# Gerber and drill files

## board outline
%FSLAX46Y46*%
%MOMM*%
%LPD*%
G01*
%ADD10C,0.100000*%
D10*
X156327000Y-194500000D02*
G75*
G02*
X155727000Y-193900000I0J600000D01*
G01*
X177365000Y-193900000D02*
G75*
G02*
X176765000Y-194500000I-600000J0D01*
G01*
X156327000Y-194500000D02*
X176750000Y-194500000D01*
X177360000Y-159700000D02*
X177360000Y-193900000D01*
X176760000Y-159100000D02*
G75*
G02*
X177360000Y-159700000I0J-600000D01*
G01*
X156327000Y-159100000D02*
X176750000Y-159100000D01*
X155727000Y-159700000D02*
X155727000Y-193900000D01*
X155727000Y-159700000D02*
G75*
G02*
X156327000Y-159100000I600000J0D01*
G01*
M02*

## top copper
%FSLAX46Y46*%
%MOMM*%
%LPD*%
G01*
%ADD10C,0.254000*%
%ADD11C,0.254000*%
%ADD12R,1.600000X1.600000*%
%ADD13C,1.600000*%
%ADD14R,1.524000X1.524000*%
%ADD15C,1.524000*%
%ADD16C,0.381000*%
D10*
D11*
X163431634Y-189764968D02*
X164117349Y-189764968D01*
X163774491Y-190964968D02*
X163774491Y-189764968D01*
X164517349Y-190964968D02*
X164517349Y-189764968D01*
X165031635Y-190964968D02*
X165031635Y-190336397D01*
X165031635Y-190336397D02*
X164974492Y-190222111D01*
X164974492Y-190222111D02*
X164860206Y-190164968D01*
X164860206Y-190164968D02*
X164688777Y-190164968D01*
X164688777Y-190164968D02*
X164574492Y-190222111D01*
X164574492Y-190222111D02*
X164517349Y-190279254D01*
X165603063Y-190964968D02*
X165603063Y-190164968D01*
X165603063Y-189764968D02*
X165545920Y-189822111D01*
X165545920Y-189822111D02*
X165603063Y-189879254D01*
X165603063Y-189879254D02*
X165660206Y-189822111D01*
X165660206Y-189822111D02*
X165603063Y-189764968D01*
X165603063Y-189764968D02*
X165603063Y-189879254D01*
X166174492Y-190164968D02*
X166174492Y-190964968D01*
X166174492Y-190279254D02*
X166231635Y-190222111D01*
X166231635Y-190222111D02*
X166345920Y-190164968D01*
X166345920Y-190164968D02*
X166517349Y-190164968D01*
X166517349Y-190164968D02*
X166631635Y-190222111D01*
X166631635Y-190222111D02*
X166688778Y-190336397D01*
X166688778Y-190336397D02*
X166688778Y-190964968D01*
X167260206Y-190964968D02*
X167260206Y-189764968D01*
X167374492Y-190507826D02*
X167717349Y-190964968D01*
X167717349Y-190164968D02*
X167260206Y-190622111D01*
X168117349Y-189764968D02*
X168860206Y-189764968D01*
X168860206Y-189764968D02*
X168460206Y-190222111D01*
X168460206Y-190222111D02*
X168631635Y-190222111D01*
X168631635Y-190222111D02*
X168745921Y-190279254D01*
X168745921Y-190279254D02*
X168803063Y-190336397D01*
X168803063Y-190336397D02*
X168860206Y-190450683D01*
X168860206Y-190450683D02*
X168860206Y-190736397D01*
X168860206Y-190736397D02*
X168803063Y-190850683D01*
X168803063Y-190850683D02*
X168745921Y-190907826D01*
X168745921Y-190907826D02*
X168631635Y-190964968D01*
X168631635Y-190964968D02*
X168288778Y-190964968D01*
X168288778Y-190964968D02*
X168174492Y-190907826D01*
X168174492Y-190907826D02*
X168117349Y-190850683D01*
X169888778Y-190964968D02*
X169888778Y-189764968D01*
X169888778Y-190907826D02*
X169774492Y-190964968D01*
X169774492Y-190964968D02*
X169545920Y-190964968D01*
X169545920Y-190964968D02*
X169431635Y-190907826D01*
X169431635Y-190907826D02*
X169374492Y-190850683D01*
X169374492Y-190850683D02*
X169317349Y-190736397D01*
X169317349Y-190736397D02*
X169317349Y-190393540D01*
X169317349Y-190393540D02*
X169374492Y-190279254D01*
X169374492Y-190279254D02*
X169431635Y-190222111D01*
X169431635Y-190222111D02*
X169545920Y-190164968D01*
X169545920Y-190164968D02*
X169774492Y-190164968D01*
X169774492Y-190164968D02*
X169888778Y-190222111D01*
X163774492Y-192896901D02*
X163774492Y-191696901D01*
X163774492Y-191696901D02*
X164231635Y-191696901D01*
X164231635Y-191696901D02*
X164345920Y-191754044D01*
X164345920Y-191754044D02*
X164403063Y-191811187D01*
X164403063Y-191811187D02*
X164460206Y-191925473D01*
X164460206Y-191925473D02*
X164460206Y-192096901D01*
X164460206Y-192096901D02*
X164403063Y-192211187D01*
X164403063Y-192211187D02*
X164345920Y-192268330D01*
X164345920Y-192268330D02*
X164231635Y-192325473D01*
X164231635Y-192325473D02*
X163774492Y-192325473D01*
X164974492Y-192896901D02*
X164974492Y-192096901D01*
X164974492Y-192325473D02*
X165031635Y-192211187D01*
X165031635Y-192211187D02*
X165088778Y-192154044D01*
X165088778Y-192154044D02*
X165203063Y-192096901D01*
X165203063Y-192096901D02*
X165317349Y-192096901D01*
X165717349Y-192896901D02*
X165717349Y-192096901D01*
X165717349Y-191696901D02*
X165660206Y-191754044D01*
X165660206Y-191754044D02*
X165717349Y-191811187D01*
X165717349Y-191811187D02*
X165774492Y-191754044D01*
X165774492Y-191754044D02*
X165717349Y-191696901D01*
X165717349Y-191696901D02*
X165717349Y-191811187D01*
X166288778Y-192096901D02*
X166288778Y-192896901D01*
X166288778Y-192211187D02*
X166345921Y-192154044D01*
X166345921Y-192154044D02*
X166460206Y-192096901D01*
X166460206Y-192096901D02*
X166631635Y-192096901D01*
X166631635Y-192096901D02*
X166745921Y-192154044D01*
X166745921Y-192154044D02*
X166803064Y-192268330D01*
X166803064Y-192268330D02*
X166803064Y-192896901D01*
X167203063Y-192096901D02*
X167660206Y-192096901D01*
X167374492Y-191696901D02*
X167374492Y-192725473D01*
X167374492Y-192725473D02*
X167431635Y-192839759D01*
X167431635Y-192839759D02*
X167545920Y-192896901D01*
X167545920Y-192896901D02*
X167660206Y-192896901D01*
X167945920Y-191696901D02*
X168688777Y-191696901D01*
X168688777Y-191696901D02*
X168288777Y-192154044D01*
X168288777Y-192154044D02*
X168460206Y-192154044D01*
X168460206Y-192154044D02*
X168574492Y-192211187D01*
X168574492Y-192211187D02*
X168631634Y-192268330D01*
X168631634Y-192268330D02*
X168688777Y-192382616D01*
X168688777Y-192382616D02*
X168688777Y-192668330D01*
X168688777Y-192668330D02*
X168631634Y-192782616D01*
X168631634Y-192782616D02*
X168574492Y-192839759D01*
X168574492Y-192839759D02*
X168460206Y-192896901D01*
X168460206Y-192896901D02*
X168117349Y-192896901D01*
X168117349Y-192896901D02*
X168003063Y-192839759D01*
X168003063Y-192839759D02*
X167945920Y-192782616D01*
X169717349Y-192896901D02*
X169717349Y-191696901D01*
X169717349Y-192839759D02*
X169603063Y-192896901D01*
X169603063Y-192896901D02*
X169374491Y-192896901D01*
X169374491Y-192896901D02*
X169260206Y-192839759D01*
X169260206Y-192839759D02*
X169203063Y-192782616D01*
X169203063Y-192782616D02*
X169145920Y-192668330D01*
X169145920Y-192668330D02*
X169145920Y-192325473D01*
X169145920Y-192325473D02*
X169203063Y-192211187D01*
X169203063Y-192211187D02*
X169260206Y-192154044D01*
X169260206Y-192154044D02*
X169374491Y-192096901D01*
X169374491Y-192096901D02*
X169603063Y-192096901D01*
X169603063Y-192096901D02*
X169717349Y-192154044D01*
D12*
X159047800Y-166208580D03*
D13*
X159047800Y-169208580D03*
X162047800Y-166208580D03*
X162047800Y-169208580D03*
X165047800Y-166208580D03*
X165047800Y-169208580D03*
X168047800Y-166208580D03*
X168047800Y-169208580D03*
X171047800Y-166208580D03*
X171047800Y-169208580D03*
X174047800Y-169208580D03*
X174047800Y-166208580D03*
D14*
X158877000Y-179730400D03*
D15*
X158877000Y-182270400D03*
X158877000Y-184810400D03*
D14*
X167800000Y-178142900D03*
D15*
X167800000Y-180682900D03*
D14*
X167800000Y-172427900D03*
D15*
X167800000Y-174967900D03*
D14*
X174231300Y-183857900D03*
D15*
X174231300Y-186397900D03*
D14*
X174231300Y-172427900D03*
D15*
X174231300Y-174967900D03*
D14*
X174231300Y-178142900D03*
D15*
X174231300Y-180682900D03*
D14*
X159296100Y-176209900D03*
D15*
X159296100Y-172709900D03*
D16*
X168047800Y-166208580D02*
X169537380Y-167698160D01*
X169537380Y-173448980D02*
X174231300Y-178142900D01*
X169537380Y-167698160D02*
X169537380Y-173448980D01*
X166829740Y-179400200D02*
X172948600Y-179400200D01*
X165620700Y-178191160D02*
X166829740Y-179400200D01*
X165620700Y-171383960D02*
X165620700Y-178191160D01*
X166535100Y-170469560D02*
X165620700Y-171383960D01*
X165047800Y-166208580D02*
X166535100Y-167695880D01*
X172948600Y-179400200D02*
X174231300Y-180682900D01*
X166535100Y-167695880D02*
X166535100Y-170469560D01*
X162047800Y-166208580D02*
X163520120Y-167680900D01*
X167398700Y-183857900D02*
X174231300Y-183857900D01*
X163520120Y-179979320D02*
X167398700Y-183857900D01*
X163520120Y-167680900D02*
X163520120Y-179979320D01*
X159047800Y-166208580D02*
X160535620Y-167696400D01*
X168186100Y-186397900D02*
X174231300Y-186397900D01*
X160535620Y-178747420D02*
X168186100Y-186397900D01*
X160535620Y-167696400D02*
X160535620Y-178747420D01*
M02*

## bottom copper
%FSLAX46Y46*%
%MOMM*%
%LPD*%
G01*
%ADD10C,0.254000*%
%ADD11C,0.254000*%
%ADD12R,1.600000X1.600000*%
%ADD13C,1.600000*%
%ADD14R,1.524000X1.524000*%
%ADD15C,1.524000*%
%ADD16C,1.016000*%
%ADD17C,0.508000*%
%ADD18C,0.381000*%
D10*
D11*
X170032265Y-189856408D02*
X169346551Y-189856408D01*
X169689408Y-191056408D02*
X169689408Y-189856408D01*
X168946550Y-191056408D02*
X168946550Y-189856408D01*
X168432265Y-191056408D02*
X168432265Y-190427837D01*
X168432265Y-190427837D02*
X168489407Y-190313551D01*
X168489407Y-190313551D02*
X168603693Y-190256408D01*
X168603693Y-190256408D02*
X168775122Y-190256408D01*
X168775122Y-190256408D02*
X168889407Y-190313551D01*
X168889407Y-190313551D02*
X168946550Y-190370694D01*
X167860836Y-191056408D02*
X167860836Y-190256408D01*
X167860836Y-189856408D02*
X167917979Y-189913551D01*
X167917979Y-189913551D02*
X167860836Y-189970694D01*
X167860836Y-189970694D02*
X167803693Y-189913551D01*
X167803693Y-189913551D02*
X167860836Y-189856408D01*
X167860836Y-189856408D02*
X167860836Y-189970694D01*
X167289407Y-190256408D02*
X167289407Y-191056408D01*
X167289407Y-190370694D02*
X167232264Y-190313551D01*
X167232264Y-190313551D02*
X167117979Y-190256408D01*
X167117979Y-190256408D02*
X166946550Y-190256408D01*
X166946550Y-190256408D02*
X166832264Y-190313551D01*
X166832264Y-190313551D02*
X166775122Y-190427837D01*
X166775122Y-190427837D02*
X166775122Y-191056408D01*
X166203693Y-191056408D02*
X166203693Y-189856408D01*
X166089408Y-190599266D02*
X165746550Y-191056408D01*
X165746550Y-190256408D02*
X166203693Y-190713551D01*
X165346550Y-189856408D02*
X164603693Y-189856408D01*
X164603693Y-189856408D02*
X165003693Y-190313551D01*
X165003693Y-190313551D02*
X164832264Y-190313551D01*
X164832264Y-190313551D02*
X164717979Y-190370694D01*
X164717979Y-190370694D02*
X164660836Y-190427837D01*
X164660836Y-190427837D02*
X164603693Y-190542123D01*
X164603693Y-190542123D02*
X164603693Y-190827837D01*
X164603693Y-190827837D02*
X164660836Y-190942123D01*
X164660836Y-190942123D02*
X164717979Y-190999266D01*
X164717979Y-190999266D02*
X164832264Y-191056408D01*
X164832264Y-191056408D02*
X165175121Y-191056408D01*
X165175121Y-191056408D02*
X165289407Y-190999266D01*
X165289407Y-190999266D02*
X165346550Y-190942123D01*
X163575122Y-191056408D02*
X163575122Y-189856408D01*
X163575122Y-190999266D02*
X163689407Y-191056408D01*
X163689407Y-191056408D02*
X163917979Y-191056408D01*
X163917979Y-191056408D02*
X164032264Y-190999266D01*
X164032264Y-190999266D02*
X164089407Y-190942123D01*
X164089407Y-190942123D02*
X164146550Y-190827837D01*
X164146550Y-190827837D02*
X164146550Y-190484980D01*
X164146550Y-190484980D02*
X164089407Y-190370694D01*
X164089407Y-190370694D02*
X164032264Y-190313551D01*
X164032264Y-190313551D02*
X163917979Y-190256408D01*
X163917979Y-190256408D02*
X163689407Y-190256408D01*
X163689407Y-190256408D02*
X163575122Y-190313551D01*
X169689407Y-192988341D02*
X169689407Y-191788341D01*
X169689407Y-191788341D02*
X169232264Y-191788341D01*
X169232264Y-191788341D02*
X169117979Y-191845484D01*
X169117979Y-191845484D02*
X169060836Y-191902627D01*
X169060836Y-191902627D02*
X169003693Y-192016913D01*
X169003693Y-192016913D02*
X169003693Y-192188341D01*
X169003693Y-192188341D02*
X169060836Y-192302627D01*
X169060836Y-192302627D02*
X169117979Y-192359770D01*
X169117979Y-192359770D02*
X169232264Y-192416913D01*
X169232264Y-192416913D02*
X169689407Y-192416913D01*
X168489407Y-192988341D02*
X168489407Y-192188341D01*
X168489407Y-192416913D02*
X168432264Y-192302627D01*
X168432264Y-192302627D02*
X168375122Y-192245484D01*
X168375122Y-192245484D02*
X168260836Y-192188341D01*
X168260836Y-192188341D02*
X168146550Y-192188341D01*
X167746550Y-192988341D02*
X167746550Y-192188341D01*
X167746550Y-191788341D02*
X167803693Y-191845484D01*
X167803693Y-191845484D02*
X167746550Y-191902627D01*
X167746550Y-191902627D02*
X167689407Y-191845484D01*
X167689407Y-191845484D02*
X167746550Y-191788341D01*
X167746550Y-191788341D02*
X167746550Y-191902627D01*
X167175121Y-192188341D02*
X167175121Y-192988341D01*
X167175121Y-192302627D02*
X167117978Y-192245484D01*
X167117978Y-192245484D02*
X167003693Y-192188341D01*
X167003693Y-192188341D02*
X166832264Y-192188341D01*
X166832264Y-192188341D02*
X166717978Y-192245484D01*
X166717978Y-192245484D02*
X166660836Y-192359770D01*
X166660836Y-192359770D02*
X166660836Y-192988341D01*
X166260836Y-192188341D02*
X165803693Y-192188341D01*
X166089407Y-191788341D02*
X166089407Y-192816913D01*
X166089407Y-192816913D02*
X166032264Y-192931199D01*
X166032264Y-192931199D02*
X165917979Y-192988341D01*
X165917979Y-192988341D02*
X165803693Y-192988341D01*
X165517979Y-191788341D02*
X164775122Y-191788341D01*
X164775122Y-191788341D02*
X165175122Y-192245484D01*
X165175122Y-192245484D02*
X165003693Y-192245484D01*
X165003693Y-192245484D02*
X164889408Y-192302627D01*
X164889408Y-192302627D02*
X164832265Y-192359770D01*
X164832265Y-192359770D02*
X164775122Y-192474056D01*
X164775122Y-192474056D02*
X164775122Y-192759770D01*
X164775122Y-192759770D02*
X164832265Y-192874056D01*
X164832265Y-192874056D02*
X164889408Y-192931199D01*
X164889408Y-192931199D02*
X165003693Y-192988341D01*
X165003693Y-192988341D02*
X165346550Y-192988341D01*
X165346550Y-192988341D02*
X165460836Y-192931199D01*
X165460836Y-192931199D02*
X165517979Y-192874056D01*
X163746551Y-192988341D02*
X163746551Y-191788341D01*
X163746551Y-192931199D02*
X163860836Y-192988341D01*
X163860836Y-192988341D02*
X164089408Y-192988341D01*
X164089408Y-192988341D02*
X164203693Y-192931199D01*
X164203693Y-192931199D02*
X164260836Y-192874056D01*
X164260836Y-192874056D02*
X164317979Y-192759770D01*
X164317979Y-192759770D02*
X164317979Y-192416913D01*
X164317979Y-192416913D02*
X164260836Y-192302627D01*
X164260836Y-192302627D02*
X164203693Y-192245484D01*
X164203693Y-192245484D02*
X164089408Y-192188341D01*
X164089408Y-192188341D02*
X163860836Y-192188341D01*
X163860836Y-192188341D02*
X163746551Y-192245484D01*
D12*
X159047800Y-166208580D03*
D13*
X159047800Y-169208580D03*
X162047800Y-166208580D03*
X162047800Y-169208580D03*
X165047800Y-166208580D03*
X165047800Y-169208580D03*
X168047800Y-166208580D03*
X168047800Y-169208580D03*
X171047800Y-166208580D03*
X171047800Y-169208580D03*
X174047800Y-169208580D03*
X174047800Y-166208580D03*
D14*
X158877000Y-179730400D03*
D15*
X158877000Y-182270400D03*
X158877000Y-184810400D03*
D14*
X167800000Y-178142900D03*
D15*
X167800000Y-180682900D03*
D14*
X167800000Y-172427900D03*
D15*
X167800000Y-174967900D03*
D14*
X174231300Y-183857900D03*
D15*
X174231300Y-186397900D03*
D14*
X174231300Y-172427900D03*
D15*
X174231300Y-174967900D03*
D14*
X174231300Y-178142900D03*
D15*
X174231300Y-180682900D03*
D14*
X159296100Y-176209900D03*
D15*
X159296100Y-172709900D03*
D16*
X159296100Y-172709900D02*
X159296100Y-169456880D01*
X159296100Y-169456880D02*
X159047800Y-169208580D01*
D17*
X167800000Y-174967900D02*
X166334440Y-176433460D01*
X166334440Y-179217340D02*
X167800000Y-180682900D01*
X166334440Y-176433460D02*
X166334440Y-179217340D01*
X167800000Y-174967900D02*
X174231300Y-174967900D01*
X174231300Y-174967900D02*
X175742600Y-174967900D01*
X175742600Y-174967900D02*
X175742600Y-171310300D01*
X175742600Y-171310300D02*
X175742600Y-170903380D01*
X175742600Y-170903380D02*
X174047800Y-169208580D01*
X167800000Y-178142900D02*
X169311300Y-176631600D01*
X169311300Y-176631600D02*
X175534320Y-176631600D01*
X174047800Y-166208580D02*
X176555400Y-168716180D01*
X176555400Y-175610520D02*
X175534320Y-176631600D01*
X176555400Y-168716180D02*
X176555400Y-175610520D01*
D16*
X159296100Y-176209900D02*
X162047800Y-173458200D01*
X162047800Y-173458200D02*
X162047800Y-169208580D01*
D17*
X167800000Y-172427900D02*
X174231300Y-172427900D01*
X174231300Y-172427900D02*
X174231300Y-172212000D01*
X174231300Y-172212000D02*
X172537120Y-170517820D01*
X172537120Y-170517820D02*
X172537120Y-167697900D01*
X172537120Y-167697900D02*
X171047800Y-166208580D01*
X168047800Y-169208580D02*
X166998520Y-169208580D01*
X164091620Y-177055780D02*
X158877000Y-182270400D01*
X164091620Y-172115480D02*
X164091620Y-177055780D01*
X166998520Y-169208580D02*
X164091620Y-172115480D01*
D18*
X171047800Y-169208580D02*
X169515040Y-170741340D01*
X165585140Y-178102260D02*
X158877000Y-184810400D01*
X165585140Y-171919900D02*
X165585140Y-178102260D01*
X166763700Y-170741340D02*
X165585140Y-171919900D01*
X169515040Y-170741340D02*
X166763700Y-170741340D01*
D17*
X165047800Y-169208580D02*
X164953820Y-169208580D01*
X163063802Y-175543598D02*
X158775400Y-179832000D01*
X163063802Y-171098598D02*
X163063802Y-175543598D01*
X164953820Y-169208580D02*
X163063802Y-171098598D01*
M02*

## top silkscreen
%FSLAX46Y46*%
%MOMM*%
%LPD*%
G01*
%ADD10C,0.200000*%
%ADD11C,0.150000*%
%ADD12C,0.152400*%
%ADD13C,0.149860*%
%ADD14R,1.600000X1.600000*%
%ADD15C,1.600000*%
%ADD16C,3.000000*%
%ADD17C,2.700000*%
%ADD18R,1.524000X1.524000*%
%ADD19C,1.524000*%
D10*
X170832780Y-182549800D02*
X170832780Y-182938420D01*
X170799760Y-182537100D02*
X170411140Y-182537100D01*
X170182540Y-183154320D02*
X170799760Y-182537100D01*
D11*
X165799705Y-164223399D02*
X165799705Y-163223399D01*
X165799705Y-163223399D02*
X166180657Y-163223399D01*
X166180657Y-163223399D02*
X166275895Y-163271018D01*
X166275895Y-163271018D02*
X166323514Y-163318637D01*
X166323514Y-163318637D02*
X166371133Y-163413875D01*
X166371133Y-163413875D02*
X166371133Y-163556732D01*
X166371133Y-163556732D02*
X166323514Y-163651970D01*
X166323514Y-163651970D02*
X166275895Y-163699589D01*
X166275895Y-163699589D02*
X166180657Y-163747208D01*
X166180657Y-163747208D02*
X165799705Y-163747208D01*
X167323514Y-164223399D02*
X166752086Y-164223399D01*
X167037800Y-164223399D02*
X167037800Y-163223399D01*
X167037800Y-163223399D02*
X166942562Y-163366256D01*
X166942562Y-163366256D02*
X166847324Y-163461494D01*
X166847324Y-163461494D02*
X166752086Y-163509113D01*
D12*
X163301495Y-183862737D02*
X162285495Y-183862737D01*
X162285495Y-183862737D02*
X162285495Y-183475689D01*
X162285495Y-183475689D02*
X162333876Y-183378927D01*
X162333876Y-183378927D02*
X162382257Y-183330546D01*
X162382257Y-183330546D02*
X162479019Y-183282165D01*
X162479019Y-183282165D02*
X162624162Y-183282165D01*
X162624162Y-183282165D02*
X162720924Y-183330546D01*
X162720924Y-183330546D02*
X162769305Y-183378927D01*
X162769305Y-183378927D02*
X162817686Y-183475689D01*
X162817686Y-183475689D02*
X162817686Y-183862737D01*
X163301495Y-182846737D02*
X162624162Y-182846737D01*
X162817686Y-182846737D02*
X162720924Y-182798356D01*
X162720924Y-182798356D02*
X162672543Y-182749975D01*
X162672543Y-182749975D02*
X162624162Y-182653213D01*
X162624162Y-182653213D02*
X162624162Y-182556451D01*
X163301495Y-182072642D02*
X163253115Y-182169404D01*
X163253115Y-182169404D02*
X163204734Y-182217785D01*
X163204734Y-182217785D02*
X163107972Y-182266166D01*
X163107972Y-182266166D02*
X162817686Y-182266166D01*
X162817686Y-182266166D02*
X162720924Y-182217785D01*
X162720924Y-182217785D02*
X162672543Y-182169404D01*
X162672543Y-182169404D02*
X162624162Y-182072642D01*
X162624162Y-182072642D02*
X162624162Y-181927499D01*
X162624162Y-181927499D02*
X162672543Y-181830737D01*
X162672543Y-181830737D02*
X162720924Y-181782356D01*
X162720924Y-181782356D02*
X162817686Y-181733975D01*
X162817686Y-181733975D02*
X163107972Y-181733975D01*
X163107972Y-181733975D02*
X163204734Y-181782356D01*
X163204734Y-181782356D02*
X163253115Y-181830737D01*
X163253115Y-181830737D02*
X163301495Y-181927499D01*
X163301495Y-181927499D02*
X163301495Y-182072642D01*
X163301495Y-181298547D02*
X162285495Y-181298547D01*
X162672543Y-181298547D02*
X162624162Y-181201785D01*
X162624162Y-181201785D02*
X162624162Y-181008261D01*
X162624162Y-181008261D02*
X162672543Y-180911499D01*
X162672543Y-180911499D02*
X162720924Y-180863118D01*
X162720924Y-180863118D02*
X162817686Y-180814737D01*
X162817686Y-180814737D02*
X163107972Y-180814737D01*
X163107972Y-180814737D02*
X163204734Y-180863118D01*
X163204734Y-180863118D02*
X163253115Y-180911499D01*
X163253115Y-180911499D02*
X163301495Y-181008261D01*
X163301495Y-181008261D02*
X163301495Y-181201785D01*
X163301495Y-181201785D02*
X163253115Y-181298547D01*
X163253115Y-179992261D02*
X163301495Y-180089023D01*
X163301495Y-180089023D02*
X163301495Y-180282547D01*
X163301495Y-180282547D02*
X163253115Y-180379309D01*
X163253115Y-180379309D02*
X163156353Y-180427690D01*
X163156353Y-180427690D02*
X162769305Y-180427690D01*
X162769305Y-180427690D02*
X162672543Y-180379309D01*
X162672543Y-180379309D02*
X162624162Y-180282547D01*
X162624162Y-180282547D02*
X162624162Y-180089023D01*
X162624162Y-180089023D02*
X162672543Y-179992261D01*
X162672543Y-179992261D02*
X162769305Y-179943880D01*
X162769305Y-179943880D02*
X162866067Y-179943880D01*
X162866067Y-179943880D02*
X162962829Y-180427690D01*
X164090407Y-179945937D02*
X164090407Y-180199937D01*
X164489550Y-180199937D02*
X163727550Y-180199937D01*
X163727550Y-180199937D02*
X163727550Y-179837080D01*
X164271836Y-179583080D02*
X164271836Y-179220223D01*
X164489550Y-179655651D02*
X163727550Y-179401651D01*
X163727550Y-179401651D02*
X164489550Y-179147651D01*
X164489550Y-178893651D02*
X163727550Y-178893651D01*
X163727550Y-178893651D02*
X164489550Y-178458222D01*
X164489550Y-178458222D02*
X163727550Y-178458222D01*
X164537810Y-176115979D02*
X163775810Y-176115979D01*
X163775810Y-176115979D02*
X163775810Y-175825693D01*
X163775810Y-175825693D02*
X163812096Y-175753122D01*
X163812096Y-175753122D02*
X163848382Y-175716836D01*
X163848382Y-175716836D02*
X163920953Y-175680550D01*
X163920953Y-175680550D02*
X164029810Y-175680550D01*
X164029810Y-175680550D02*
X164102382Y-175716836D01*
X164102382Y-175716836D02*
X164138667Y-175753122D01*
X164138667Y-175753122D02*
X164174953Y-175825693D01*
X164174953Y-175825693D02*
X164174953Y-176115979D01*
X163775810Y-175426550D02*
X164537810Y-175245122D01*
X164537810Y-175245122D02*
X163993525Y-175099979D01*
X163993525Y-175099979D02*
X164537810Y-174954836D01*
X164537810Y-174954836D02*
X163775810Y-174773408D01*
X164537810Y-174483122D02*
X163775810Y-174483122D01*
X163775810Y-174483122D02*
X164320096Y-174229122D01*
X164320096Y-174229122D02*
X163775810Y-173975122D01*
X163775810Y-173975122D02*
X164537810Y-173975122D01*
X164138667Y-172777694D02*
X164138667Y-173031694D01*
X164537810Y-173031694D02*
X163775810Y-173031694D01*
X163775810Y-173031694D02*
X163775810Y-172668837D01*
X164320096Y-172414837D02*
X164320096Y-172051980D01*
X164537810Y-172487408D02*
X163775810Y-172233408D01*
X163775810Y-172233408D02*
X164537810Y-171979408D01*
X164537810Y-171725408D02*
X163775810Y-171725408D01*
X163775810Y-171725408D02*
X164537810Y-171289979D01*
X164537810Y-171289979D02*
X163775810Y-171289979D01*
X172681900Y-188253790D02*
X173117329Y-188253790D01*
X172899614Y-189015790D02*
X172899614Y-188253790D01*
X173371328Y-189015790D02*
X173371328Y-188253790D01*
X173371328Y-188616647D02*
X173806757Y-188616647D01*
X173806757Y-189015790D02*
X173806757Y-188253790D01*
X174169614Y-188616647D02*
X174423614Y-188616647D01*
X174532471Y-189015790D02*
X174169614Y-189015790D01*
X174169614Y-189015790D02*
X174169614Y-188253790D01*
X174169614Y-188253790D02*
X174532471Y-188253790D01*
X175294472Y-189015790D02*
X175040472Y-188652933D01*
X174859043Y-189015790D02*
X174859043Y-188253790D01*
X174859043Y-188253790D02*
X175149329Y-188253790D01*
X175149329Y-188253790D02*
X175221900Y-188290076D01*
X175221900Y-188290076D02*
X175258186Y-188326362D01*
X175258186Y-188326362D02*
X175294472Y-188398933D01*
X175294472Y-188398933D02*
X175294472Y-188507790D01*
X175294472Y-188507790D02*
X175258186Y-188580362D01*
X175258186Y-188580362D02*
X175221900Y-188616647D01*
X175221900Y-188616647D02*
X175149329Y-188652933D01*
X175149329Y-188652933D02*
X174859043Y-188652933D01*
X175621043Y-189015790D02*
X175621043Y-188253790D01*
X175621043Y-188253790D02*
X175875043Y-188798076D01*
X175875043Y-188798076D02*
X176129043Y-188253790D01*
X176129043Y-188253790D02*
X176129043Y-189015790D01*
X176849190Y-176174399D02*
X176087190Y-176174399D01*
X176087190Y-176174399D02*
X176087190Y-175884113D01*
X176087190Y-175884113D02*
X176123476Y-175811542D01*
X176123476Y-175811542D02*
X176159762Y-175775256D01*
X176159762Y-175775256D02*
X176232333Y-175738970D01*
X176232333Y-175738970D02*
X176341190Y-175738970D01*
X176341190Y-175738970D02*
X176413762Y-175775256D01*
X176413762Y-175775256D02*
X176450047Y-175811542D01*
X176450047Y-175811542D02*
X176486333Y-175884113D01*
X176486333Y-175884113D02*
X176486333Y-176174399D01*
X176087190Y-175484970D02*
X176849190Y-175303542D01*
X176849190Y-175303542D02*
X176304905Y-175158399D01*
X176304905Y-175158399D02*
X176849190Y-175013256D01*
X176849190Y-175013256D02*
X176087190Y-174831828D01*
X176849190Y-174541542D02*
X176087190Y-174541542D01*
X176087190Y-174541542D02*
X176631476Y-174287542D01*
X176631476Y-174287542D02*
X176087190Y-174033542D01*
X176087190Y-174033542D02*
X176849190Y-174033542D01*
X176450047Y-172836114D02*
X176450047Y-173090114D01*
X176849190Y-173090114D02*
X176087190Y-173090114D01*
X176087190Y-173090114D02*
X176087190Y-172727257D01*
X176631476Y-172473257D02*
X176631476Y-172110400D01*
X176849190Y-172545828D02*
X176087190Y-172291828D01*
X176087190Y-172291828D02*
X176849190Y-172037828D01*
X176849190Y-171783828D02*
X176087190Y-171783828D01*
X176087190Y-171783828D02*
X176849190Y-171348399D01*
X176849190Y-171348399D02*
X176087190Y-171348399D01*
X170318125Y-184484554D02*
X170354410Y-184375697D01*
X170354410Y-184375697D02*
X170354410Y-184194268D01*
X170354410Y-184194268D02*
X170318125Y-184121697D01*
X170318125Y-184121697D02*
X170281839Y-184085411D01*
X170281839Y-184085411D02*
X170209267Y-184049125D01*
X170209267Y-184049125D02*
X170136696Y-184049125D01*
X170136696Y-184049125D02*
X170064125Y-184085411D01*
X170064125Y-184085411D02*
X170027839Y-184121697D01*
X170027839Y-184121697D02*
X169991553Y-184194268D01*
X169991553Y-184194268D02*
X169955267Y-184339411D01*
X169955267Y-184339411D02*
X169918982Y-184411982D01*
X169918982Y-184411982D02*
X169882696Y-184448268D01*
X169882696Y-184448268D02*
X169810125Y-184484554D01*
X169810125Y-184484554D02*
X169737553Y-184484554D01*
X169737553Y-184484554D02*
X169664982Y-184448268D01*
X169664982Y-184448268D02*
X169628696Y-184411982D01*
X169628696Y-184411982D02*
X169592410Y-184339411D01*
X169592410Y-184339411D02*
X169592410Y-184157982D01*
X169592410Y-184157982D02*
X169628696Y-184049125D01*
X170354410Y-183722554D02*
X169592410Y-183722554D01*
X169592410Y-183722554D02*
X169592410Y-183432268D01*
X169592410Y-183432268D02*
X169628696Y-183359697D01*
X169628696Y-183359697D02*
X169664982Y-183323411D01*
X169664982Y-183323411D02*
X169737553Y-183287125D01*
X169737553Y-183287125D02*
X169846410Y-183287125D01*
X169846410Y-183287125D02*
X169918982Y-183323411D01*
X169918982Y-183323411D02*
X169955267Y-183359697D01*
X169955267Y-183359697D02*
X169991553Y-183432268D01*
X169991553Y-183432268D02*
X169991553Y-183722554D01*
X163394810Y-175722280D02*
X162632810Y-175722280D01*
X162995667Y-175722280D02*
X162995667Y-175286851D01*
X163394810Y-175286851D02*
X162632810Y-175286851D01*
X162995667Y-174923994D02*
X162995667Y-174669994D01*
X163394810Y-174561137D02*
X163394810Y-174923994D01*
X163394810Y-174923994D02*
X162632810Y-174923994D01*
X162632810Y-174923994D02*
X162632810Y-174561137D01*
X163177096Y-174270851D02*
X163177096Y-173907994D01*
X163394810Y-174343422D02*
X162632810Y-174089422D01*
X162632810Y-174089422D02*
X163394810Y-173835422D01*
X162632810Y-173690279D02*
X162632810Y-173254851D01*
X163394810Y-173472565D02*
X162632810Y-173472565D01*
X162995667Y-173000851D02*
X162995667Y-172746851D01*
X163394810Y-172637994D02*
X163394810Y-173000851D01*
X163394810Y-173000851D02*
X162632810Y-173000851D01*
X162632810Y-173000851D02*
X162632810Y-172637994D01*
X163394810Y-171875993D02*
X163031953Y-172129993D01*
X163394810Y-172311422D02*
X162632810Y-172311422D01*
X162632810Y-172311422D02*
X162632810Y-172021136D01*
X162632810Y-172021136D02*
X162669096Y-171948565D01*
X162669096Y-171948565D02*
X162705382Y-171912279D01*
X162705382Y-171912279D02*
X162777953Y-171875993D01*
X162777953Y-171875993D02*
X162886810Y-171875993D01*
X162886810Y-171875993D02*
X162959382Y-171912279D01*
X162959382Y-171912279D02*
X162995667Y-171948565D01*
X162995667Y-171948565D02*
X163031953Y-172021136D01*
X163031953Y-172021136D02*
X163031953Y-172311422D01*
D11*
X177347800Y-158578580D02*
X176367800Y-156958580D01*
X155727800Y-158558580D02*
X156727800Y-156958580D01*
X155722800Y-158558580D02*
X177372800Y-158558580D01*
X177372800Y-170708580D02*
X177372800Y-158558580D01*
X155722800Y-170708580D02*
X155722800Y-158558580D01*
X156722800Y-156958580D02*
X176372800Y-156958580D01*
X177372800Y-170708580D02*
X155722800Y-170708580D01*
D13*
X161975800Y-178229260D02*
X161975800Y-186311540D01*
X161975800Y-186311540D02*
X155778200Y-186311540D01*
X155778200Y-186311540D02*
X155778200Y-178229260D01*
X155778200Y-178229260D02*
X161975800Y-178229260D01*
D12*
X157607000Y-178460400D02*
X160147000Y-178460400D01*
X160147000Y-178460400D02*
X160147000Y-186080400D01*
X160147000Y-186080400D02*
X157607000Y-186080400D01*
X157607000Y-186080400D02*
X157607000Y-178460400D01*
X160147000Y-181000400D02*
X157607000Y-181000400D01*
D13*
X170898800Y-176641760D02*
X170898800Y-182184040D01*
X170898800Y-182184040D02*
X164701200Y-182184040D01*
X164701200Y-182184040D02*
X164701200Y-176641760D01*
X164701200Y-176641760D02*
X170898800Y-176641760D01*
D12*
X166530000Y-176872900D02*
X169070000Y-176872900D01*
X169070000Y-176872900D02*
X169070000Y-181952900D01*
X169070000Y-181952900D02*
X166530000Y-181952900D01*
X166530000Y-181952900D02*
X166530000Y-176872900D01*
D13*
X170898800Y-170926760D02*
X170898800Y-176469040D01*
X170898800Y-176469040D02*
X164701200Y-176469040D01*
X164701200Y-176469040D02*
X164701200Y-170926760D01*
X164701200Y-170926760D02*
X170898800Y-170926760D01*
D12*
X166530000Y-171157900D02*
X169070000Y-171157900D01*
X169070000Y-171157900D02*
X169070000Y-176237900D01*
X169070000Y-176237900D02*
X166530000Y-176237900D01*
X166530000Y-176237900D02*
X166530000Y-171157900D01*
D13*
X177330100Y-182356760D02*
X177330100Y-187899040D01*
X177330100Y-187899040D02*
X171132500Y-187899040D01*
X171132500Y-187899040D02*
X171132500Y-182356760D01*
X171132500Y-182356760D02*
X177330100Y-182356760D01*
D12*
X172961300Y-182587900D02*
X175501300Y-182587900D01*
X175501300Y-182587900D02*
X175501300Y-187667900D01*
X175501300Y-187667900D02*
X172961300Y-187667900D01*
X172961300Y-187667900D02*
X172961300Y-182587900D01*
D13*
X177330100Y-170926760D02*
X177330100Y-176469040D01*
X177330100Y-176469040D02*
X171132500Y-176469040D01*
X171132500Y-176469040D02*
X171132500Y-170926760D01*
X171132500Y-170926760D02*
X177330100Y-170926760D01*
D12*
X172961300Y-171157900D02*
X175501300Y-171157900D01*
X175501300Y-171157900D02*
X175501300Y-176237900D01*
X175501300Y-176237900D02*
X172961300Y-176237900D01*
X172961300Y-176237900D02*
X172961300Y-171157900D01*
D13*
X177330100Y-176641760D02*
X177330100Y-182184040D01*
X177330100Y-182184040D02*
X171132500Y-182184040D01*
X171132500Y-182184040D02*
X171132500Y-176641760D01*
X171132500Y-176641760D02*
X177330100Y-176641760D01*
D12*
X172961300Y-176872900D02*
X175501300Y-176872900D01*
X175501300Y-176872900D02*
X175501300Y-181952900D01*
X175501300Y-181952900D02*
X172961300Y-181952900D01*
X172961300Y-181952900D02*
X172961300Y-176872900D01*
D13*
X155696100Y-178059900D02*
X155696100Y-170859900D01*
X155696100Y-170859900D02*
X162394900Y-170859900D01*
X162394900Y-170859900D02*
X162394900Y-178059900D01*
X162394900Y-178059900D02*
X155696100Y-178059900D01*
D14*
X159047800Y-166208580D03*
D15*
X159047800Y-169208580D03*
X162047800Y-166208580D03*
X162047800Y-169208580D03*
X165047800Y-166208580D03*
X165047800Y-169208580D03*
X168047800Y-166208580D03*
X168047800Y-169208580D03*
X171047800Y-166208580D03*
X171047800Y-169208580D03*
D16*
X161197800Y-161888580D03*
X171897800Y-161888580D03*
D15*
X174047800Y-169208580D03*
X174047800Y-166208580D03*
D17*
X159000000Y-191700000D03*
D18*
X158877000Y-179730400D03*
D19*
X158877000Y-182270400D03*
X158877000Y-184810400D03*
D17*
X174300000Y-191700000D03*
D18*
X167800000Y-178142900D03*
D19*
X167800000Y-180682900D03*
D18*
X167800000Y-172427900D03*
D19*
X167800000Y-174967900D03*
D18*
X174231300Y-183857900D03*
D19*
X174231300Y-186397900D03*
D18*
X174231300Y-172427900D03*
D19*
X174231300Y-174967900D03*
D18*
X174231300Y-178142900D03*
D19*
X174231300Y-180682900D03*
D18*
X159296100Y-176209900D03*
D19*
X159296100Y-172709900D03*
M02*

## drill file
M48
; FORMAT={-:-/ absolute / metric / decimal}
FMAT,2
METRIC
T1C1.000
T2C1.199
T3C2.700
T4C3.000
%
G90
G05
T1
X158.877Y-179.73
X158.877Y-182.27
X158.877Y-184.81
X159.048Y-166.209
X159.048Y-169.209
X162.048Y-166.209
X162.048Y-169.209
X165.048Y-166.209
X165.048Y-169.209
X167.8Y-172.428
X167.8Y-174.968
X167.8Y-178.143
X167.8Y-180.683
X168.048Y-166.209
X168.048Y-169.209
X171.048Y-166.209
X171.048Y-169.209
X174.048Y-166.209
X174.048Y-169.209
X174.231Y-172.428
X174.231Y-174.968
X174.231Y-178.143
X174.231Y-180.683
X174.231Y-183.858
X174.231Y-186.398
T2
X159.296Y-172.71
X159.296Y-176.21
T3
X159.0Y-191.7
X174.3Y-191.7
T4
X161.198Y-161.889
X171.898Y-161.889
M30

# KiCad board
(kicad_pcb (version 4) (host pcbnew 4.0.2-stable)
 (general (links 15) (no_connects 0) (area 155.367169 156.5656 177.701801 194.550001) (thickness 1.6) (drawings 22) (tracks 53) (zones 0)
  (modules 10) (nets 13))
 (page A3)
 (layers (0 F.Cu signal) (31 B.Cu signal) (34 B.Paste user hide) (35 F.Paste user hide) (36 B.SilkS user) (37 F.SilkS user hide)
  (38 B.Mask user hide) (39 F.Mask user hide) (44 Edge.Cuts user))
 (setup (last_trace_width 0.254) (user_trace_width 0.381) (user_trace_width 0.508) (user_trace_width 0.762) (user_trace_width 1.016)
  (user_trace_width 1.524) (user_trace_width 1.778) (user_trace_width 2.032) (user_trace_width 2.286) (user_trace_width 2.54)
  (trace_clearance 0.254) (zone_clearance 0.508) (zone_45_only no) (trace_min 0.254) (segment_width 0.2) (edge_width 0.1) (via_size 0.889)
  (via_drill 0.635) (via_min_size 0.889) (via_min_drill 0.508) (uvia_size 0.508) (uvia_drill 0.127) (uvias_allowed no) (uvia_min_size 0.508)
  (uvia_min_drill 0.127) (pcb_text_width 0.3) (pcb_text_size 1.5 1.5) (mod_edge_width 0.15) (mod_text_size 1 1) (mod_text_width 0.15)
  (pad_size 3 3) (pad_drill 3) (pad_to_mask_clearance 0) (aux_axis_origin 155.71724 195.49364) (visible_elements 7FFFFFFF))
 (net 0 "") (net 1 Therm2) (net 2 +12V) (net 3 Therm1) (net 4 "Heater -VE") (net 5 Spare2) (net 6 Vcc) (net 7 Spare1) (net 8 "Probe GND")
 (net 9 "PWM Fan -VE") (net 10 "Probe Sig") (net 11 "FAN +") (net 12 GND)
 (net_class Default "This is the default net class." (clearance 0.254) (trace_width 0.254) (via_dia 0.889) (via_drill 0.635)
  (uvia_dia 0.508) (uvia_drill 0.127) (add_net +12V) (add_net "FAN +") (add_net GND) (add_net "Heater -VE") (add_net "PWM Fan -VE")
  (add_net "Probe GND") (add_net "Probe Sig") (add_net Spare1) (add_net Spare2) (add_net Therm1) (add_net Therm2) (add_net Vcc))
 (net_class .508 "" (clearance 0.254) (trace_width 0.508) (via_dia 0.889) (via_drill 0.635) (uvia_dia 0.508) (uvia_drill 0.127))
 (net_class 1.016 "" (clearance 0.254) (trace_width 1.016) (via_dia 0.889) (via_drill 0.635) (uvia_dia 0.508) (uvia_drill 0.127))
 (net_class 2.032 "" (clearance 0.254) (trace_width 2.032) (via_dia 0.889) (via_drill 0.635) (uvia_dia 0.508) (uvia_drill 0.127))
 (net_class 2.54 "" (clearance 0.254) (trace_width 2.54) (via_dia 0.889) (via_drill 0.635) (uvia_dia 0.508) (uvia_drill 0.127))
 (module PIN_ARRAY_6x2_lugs (layer F.Cu) (at 166.5478 167.70858)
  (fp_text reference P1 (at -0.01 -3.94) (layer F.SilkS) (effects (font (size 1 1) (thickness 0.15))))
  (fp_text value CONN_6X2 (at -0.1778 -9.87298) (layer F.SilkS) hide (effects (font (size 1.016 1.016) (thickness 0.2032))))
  (fp_line (start 10.8 -9.13) (end 9.82 -10.75) (layer F.SilkS) (width 0.15))
  (fp_line (start -10.82 -9.15) (end -9.82 -10.75) (layer F.SilkS) (width 0.15))
  (fp_line (start -10.825 -9.15) (end 10.825 -9.15) (layer F.SilkS) (width 0.15))
  (fp_line (start 10.825 3) (end 10.825 -9.15) (layer F.SilkS) (width 0.15))
  (fp_line (start -10.825 3) (end -10.825 -9.15) (layer F.SilkS) (width 0.15))
  (fp_line (start -9.825 -10.75) (end 9.825 -10.75) (layer F.SilkS) (width 0.15))
  (fp_line (start 10.825 3) (end -10.825 3) (layer F.SilkS) (width 0.15))
  (pad 1 thru_hole rect (at -7.5 -1.5) (size 1.6 1.6) (drill 1) (layers *.Cu *.Mask F.SilkS) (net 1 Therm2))
  (pad 2 thru_hole circle (at -7.5 1.5) (size 1.6 1.6) (drill 1) (layers *.Cu *.Mask F.SilkS) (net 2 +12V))
  (pad 3 thru_hole circle (at -4.5 -1.5) (size 1.6 1.6) (drill 1) (layers *.Cu *.Mask F.SilkS) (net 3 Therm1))
  (pad 4 thru_hole circle (at -4.5 1.5) (size 1.6 1.6) (drill 1) (layers *.Cu *.Mask F.SilkS) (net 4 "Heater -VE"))
  (pad 5 thru_hole circle (at -1.5 -1.5) (size 1.6 1.6) (drill 1) (layers *.Cu *.Mask F.SilkS) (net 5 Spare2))
  (pad 6 thru_hole circle (at -1.5 1.5) (size 1.6 1.6) (drill 1) (layers *.Cu *.Mask F.SilkS) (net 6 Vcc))
  (pad 7 thru_hole circle (at 1.5 -1.5) (size 1.6 1.6) (drill 1) (layers *.Cu *.Mask F.SilkS) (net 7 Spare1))
  (pad 8 thru_hole circle (at 1.5 1.5) (size 1.6 1.6) (drill 1) (layers *.Cu *.Mask F.SilkS) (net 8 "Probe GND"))
  (pad 9 thru_hole circle (at 4.5 -1.5) (size 1.6 1.6) (drill 1) (layers *.Cu *.Mask F.SilkS) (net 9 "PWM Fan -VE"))
  (pad 10 thru_hole circle (at 4.5 1.5) (size 1.6 1.6) (drill 1) (layers *.Cu *.Mask F.SilkS) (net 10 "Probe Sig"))
  (pad "" np_thru_hole circle (at -5.35 -5.82) (size 3 3) (drill 3) (layers *.Cu *.Mask F.SilkS))
  (pad "" np_thru_hole circle (at 5.35 -5.82) (size 3 3) (drill 3) (layers *.Cu *.Mask F.SilkS))
  (pad 12 thru_hole circle (at 7.5 1.5) (size 1.6 1.6) (drill 1) (layers *.Cu *.Mask F.SilkS) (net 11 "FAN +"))
  (pad 11 thru_hole circle (at 7.5 -1.5) (size 1.6 1.6) (drill 1) (layers *.Cu *.Mask F.SilkS) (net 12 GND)))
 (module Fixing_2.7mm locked (layer F.Cu) (at 160 191.7)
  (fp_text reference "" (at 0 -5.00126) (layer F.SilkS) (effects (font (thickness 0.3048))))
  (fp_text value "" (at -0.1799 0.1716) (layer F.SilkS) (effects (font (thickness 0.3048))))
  (pad "" np_thru_hole circle (at -1 0) (size 2.7 2.7) (drill 2.7) (layers *.Cu *.Mask F.SilkS)))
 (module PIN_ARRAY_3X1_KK (layer F.Cu) (at 158.877 182.2704 270)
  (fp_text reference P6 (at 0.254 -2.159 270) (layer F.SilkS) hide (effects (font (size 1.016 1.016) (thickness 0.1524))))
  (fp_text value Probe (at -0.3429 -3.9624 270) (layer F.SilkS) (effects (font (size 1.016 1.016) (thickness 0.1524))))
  (fp_line (start -4.04114 -3.0988) (end 4.04114 -3.0988) (layer F.SilkS) (width 0.14986))
  (fp_line (start 4.04114 -3.0988) (end 4.04114 3.0988) (layer F.SilkS) (width 0.14986))
  (fp_line (start 4.04114 3.0988) (end -4.04114 3.0988) (layer F.SilkS) (width 0.14986))
  (fp_line (start -4.04114 3.0988) (end -4.04114 -3.0988) (layer F.SilkS) (width 0.14986))
  (fp_line (start -3.81 1.27) (end -3.81 -1.27) (layer F.SilkS) (width 0.1524))
  (fp_line (start -3.81 -1.27) (end 3.81 -1.27) (layer F.SilkS) (width 0.1524))
  (fp_line (start 3.81 -1.27) (end 3.81 1.27) (layer F.SilkS) (width 0.1524))
  (fp_line (start 3.81 1.27) (end -3.81 1.27) (layer F.SilkS) (width 0.1524))
  (fp_line (start -1.27 -1.27) (end -1.27 1.27) (layer F.SilkS) (width 0.1524))
  (pad 1 thru_hole rect (at -2.54 0 270) (size 1.524 1.524) (drill 1) (layers *.Cu *.Mask F.SilkS) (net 6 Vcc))
  (pad 2 thru_hole circle (at 0 0 270) (size 1.524 1.524) (drill 1) (layers *.Cu *.Mask F.SilkS) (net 8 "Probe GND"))
  (pad 3 thru_hole circle (at 2.54 0 270) (size 1.524 1.524) (drill 1) (layers *.Cu *.Mask F.SilkS) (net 10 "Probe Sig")))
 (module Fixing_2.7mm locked (layer F.Cu) (at 174.3 191.7)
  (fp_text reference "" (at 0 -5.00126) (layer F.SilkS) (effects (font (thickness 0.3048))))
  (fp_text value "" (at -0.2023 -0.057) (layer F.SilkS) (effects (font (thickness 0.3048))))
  (pad "" np_thru_hole circle (at 0 0) (size 2.7 2.7) (drill 2.7) (layers *.Cu *.Mask F.SilkS)))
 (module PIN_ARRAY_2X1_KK (layer F.Cu) (at 167.8 179.4129 270)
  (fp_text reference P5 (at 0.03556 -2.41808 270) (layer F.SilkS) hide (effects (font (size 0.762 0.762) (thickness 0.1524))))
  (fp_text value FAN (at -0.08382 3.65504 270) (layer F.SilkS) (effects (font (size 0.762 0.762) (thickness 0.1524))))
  (fp_line (start -2.77114 -3.0988) (end 2.77114 -3.0988) (layer F.SilkS) (width 0.14986))
  (fp_line (start 2.77114 -3.0988) (end 2.77114 3.0988) (layer F.SilkS) (width 0.14986))
  (fp_line (start 2.77114 3.0988) (end -2.77114 3.0988) (layer F.SilkS) (width 0.14986))
  (fp_line (start -2.77114 3.0988) (end -2.77114 -3.0988) (layer F.SilkS) (width 0.14986))
  (fp_line (start -2.54 1.27) (end -2.54 -1.27) (layer F.SilkS) (width 0.1524))
  (fp_line (start -2.54 -1.27) (end 2.54 -1.27) (layer F.SilkS) (width 0.1524))
  (fp_line (start 2.54 -1.27) (end 2.54 1.27) (layer F.SilkS) (width 0.1524))
  (fp_line (start 2.54 1.27) (end -2.54 1.27) (layer F.SilkS) (width 0.1524))
  (pad 1 thru_hole rect (at -1.27 0 270) (size 1.524 1.524) (drill 1) (layers *.Cu *.Mask F.SilkS) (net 12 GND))
  (pad 2 thru_hole circle (at 1.27 0 270) (size 1.524 1.524) (drill 1) (layers *.Cu *.Mask F.SilkS) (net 11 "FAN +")))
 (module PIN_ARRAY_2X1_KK (layer F.Cu) (at 167.8 173.6979 270)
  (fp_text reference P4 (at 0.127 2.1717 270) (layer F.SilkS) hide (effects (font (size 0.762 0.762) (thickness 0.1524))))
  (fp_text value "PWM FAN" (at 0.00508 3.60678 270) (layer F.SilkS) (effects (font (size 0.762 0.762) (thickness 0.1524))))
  (fp_line (start -2.77114 -3.0988) (end 2.77114 -3.0988) (layer F.SilkS) (width 0.14986))
  (fp_line (start 2.77114 -3.0988) (end 2.77114 3.0988) (layer F.SilkS) (width 0.14986))
  (fp_line (start 2.77114 3.0988) (end -2.77114 3.0988) (layer F.SilkS) (width 0.14986))
  (fp_line (start -2.77114 3.0988) (end -2.77114 -3.0988) (layer F.SilkS) (width 0.14986))
  (fp_line (start -2.54 1.27) (end -2.54 -1.27) (layer F.SilkS) (width 0.1524))
  (fp_line (start -2.54 -1.27) (end 2.54 -1.27) (layer F.SilkS) (width 0.1524))
  (fp_line (start 2.54 -1.27) (end 2.54 1.27) (layer F.SilkS) (width 0.1524))
  (fp_line (start 2.54 1.27) (end -2.54 1.27) (layer F.SilkS) (width 0.1524))
  (pad 1 thru_hole rect (at -1.27 0 270) (size 1.524 1.524) (drill 1) (layers *.Cu *.Mask F.SilkS) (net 9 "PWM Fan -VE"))
  (pad 2 thru_hole circle (at 1.27 0 270) (size 1.524 1.524) (drill 1) (layers *.Cu *.Mask F.SilkS) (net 11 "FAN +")))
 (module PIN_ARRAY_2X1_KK (layer F.Cu) (at 174.2313 185.1279 270)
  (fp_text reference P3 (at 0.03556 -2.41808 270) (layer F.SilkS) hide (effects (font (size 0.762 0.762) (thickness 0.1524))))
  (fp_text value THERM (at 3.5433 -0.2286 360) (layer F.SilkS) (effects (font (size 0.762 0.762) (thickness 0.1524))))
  (fp_line (start -2.77114 -3.0988) (end 2.77114 -3.0988) (layer F.SilkS) (width 0.14986))
  (fp_line (start 2.77114 -3.0988) (end 2.77114 3.0988) (layer F.SilkS) (width 0.14986))
  (fp_line (start 2.77114 3.0988) (end -2.77114 3.0988) (layer F.SilkS) (width 0.14986))
  (fp_line (start -2.77114 3.0988) (end -2.77114 -3.0988) (layer F.SilkS) (width 0.14986))
  (fp_line (start -2.54 1.27) (end -2.54 -1.27) (layer F.SilkS) (width 0.1524))
  (fp_line (start -2.54 -1.27) (end 2.54 -1.27) (layer F.SilkS) (width 0.1524))
  (fp_line (start 2.54 -1.27) (end 2.54 1.27) (layer F.SilkS) (width 0.1524))
  (fp_line (start 2.54 1.27) (end -2.54 1.27) (layer F.SilkS) (width 0.1524))
  (pad 1 thru_hole rect (at -1.27 0 270) (size 1.524 1.524) (drill 1) (layers *.Cu *.Mask F.SilkS) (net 3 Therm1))
  (pad 2 thru_hole circle (at 1.27 0 270) (size 1.524 1.524) (drill 1) (layers *.Cu *.Mask F.SilkS) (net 1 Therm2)))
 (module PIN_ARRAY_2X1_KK (layer F.Cu) (at 174.2313 173.6979 270)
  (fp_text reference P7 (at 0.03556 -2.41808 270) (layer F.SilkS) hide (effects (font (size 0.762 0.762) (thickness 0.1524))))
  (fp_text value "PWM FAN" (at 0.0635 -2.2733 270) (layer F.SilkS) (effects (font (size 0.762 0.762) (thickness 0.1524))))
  (fp_line (start -2.77114 -3.0988) (end 2.77114 -3.0988) (layer F.SilkS) (width 0.14986))
  (fp_line (start 2.77114 -3.0988) (end 2.77114 3.0988) (layer F.SilkS) (width 0.14986))
  (fp_line (start 2.77114 3.0988) (end -2.77114 3.0988) (layer F.SilkS) (width 0.14986))
  (fp_line (start -2.77114 3.0988) (end -2.77114 -3.0988) (layer F.SilkS) (width 0.14986))
  (fp_line (start -2.54 1.27) (end -2.54 -1.27) (layer F.SilkS) (width 0.1524))
  (fp_line (start -2.54 -1.27) (end 2.54 -1.27) (layer F.SilkS) (width 0.1524))
  (fp_line (start 2.54 -1.27) (end 2.54 1.27) (layer F.SilkS) (width 0.1524))
  (fp_line (start 2.54 1.27) (end -2.54 1.27) (layer F.SilkS) (width 0.1524))
  (pad 1 thru_hole rect (at -1.27 0 270) (size 1.524 1.524) (drill 1) (layers *.Cu *.Mask F.SilkS) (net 9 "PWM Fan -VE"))
  (pad 2 thru_hole circle (at 1.27 0 270) (size 1.524 1.524) (drill 1) (layers *.Cu *.Mask F.SilkS) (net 11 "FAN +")))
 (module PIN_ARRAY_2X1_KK (layer F.Cu) (at 174.2313 179.4129 270)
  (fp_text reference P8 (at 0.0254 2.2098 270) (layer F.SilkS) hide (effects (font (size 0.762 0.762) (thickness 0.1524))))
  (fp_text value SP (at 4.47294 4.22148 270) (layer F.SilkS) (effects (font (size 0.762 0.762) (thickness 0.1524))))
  (fp_line (start -2.77114 -3.0988) (end 2.77114 -3.0988) (layer F.SilkS) (width 0.14986))
  (fp_line (start 2.77114 -3.0988) (end 2.77114 3.0988) (layer F.SilkS) (width 0.14986))
  (fp_line (start 2.77114 3.0988) (end -2.77114 3.0988) (layer F.SilkS) (width 0.14986))
  (fp_line (start -2.77114 3.0988) (end -2.77114 -3.0988) (layer F.SilkS) (width 0.14986))
  (fp_line (start -2.54 1.27) (end -2.54 -1.27) (layer F.SilkS) (width 0.1524))
  (fp_line (start -2.54 -1.27) (end 2.54 -1.27) (layer F.SilkS) (width 0.1524))
  (fp_line (start 2.54 -1.27) (end 2.54 1.27) (layer F.SilkS) (width 0.1524))
  (fp_line (start 2.54 1.27) (end -2.54 1.27) (layer F.SilkS) (width 0.1524))
  (pad 1 thru_hole rect (at -1.27 0 270) (size 1.524 1.524) (drill 1) (layers *.Cu *.Mask F.SilkS) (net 7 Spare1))
  (pad 2 thru_hole circle (at 1.27 0 270) (size 1.524 1.524) (drill 1) (layers *.Cu *.Mask F.SilkS) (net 5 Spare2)))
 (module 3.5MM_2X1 (layer F.Cu) (at 159.2961 174.4599 90)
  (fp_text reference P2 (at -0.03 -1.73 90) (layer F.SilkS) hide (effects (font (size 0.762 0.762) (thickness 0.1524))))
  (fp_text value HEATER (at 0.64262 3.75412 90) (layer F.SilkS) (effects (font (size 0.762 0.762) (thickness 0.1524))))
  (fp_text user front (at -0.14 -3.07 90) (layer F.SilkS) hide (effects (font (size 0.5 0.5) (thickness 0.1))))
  (fp_line (start -3.6 -3.6) (end 3.6 -3.6) (layer F.SilkS) (width 0.14986))
  (fp_line (start 3.6 -3.6) (end 3.6 3.0988) (layer F.SilkS) (width 0.14986))
  (fp_line (start 3.6 3.0988) (end -3.6 3.0988) (layer F.SilkS) (width 0.14986))
  (fp_line (start -3.6 3.0988) (end -3.6 -3.6) (layer F.SilkS) (width 0.14986))
  (pad 1 thru_hole rect (at -1.75 0 90) (size 1.524 1.524) (drill 1.19888) (layers *.Cu *.Mask F.SilkS) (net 4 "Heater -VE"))
  (pad 2 thru_hole circle (at 1.75 0 90) (size 1.524 1.524) (drill 1.19888) (layers *.Cu *.Mask F.SilkS) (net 2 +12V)))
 (gr_line (start 170.83278 182.5498) (end 170.83278 182.93842) (angle 90) (layer F.SilkS) (width 0.2))
 (gr_line (start 170.79976 182.5371) (end 170.41114 182.5371) (angle 90) (layer F.SilkS) (width 0.2))
 (gr_line (start 170.18254 183.15432) (end 170.79976 182.5371) (angle 90) (layer F.SilkS) (width 0.2))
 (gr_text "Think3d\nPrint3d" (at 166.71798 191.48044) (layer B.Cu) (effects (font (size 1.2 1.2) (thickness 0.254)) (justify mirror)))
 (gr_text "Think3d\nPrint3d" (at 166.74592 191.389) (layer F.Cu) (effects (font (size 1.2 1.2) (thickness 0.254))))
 (gr_arc (start 156.327 193.9) (end 156.327 194.5) (angle 90) (layer Edge.Cuts) (width 0.1))
 (gr_arc (start 176.765 193.9) (end 177.365 193.9) (angle 90) (layer Edge.Cuts) (width 0.1))
 (gr_line (start 156.327 194.5) (end 176.75 194.5) (angle 90) (layer Edge.Cuts) (width 0.1))
 (gr_line (start 177.36 159.7) (end 177.36 193.9) (angle 90) (layer Edge.Cuts) (width 0.1))
 (gr_arc (start 176.76 159.7) (end 176.76 159.1) (angle 90) (layer Edge.Cuts) (width 0.1))
 (gr_line (start 156.327 159.1) (end 176.75 159.1) (angle 90) (layer Edge.Cuts) (width 0.1))
 (gr_line (start 155.727 159.7) (end 155.727 193.9) (angle 90) (layer Edge.Cuts) (width 0.1))
 (gr_arc (start 156.327 159.7) (end 155.727 159.7) (angle 90) (layer Edge.Cuts) (width 0.1))
 (segment (start 159.2961 172.7099) (end 159.2961 169.45688) (width 1.016) (layer B.Cu) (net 2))
 (segment (start 159.2961 169.45688) (end 159.0478 169.20858) (width 1.016) (layer B.Cu) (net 2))
 (segment (start 167.8 174.9679) (end 166.33444 176.43346) (width 0.508) (layer B.Cu) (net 11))
 (segment (start 166.33444 179.21734) (end 167.8 180.6829) (width 0.508) (layer B.Cu) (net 11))
 (segment (start 166.33444 176.43346) (end 166.33444 179.21734) (width 0.508) (layer B.Cu) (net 11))
 (segment (start 167.8 174.9679) (end 174.2313 174.9679) (width 0.508) (layer B.Cu) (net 11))
 (segment (start 174.2313 174.9679) (end 175.7426 174.9679) (width 0.508) (layer B.Cu) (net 11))
 (segment (start 175.7426 174.9679) (end 175.7426 171.3103) (width 0.508) (layer B.Cu) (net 11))
 (segment (start 175.7426 171.3103) (end 175.7426 170.90338) (width 0.508) (layer B.Cu) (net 11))
 (segment (start 175.7426 170.90338) (end 174.0478 169.20858) (width 0.508) (layer B.Cu) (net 11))
 (segment (start 167.8 178.1429) (end 169.3113 176.6316) (width 0.508) (layer B.Cu) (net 12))
 (segment (start 169.3113 176.6316) (end 175.53432 176.6316) (width 0.508) (layer B.Cu) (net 12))
 (segment (start 174.0478 166.20858) (end 176.5554 168.71618) (width 0.508) (layer B.Cu) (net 12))
 (segment (start 176.5554 175.61052) (end 175.53432 176.6316) (width 0.508) (layer B.Cu) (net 12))
 (segment (start 176.5554 168.71618) (end 176.5554 175.61052) (width 0.508) (layer B.Cu) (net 12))
 (segment (start 159.2961 176.2099) (end 162.0478 173.4582) (width 1.016) (layer B.Cu) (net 4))
 (segment (start 162.0478 173.4582) (end 162.0478 169.20858) (width 1.016) (layer B.Cu) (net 4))
 (segment (start 167.8 172.4279) (end 174.2313 172.4279) (width 0.508) (layer B.Cu) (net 9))
 (segment (start 174.2313 172.4279) (end 174.2313 172.212) (width 0.508) (layer B.Cu) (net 9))
 (segment (start 174.2313 172.212) (end 172.53712 170.51782) (width 0.508) (layer B.Cu) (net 9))
 (segment (start 172.53712 170.51782) (end 172.53712 167.6979) (width 0.508) (layer B.Cu) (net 9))
 (segment (start 172.53712 167.6979) (end 171.0478 166.20858) (width 0.508) (layer B.Cu) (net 9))
 (segment (start 168.0478 169.20858) (end 166.99852 169.20858) (width 0.508) (layer B.Cu) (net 8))
 (segment (start 164.09162 177.05578) (end 158.877 182.2704) (width 0.508) (layer B.Cu) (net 8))
 (segment (start 164.09162 172.11548) (end 164.09162 177.05578) (width 0.508) (layer B.Cu) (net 8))
 (segment (start 166.99852 169.20858) (end 164.09162 172.11548) (width 0.508) (layer B.Cu) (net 8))
 (segment (start 171.0478 169.20858) (end 169.51504 170.74134) (width 0.381) (layer B.Cu) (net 10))
 (segment (start 165.58514 178.10226) (end 158.877 184.8104) (width 0.381) (layer B.Cu) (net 10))
 (segment (start 165.58514 171.9199) (end 165.58514 178.10226) (width 0.381) (layer B.Cu) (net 10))
 (segment (start 166.7637 170.74134) (end 165.58514 171.9199) (width 0.381) (layer B.Cu) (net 10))
 (segment (start 169.51504 170.74134) (end 166.7637 170.74134) (width 0.381) (layer B.Cu) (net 10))
 (segment (start 168.0478 166.20858) (end 169.53738 167.69816) (width 0.381) (layer F.Cu) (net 7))
 (segment (start 169.53738 173.44898) (end 174.2313 178.1429) (width 0.381) (layer F.Cu) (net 7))
 (segment (start 169.53738 167.69816) (end 169.53738 173.44898) (width 0.381) (layer F.Cu) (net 7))
 (segment (start 166.82974 179.4002) (end 172.9486 179.4002) (width 0.381) (layer F.Cu) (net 5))
 (segment (start 165.6207 178.19116) (end 166.82974 179.4002) (width 0.381) (layer F.Cu) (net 5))
 (segment (start 165.6207 171.38396) (end 165.6207 178.19116) (width 0.381) (layer F.Cu) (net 5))
 (segment (start 166.5351 170.46956) (end 165.6207 171.38396) (width 0.381) (layer F.Cu) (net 5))
 (segment (start 165.0478 166.20858) (end 166.5351 167.69588) (width 0.381) (layer F.Cu) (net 5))
 (segment (start 172.9486 179.4002) (end 174.2313 180.6829) (width 0.381) (layer F.Cu) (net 5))
 (segment (start 166.5351 167.69588) (end 166.5351 170.46956) (width 0.381) (layer F.Cu) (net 5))
 (segment (start 162.0478 166.20858) (end 163.52012 167.6809) (width 0.381) (layer F.Cu) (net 3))
 (segment (start 167.3987 183.8579) (end 174.2313 183.8579) (width 0.381) (layer F.Cu) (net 3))
 (segment (start 163.52012 179.97932) (end 167.3987 183.8579) (width 0.381) (layer F.Cu) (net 3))
 (segment (start 163.52012 167.6809) (end 163.52012 179.97932) (width 0.381) (layer F.Cu) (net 3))
 (segment (start 159.0478 166.20858) (end 160.53562 167.6964) (width 0.381) (layer F.Cu) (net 1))
 (segment (start 168.1861 186.3979) (end 174.2313 186.3979) (width 0.381) (layer F.Cu) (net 1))
 (segment (start 160.53562 178.74742) (end 168.1861 186.3979) (width 0.381) (layer F.Cu) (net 1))
 (segment (start 160.53562 167.6964) (end 160.53562 178.74742) (width 0.381) (layer F.Cu) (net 1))
 (segment (start 165.0478 169.20858) (end 164.95382 169.20858) (width 0.508) (layer B.Cu) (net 6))
 (segment (start 163.063802 175.543598) (end 158.7754 179.832) (width 0.508) (layer B.Cu) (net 6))
 (segment (start 163.063802 171.098598) (end 163.063802 175.543598) (width 0.508) (layer B.Cu) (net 6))
 (segment (start 164.95382 169.20858) (end 163.063802 171.098598) (width 0.508) (layer B.Cu) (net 6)))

